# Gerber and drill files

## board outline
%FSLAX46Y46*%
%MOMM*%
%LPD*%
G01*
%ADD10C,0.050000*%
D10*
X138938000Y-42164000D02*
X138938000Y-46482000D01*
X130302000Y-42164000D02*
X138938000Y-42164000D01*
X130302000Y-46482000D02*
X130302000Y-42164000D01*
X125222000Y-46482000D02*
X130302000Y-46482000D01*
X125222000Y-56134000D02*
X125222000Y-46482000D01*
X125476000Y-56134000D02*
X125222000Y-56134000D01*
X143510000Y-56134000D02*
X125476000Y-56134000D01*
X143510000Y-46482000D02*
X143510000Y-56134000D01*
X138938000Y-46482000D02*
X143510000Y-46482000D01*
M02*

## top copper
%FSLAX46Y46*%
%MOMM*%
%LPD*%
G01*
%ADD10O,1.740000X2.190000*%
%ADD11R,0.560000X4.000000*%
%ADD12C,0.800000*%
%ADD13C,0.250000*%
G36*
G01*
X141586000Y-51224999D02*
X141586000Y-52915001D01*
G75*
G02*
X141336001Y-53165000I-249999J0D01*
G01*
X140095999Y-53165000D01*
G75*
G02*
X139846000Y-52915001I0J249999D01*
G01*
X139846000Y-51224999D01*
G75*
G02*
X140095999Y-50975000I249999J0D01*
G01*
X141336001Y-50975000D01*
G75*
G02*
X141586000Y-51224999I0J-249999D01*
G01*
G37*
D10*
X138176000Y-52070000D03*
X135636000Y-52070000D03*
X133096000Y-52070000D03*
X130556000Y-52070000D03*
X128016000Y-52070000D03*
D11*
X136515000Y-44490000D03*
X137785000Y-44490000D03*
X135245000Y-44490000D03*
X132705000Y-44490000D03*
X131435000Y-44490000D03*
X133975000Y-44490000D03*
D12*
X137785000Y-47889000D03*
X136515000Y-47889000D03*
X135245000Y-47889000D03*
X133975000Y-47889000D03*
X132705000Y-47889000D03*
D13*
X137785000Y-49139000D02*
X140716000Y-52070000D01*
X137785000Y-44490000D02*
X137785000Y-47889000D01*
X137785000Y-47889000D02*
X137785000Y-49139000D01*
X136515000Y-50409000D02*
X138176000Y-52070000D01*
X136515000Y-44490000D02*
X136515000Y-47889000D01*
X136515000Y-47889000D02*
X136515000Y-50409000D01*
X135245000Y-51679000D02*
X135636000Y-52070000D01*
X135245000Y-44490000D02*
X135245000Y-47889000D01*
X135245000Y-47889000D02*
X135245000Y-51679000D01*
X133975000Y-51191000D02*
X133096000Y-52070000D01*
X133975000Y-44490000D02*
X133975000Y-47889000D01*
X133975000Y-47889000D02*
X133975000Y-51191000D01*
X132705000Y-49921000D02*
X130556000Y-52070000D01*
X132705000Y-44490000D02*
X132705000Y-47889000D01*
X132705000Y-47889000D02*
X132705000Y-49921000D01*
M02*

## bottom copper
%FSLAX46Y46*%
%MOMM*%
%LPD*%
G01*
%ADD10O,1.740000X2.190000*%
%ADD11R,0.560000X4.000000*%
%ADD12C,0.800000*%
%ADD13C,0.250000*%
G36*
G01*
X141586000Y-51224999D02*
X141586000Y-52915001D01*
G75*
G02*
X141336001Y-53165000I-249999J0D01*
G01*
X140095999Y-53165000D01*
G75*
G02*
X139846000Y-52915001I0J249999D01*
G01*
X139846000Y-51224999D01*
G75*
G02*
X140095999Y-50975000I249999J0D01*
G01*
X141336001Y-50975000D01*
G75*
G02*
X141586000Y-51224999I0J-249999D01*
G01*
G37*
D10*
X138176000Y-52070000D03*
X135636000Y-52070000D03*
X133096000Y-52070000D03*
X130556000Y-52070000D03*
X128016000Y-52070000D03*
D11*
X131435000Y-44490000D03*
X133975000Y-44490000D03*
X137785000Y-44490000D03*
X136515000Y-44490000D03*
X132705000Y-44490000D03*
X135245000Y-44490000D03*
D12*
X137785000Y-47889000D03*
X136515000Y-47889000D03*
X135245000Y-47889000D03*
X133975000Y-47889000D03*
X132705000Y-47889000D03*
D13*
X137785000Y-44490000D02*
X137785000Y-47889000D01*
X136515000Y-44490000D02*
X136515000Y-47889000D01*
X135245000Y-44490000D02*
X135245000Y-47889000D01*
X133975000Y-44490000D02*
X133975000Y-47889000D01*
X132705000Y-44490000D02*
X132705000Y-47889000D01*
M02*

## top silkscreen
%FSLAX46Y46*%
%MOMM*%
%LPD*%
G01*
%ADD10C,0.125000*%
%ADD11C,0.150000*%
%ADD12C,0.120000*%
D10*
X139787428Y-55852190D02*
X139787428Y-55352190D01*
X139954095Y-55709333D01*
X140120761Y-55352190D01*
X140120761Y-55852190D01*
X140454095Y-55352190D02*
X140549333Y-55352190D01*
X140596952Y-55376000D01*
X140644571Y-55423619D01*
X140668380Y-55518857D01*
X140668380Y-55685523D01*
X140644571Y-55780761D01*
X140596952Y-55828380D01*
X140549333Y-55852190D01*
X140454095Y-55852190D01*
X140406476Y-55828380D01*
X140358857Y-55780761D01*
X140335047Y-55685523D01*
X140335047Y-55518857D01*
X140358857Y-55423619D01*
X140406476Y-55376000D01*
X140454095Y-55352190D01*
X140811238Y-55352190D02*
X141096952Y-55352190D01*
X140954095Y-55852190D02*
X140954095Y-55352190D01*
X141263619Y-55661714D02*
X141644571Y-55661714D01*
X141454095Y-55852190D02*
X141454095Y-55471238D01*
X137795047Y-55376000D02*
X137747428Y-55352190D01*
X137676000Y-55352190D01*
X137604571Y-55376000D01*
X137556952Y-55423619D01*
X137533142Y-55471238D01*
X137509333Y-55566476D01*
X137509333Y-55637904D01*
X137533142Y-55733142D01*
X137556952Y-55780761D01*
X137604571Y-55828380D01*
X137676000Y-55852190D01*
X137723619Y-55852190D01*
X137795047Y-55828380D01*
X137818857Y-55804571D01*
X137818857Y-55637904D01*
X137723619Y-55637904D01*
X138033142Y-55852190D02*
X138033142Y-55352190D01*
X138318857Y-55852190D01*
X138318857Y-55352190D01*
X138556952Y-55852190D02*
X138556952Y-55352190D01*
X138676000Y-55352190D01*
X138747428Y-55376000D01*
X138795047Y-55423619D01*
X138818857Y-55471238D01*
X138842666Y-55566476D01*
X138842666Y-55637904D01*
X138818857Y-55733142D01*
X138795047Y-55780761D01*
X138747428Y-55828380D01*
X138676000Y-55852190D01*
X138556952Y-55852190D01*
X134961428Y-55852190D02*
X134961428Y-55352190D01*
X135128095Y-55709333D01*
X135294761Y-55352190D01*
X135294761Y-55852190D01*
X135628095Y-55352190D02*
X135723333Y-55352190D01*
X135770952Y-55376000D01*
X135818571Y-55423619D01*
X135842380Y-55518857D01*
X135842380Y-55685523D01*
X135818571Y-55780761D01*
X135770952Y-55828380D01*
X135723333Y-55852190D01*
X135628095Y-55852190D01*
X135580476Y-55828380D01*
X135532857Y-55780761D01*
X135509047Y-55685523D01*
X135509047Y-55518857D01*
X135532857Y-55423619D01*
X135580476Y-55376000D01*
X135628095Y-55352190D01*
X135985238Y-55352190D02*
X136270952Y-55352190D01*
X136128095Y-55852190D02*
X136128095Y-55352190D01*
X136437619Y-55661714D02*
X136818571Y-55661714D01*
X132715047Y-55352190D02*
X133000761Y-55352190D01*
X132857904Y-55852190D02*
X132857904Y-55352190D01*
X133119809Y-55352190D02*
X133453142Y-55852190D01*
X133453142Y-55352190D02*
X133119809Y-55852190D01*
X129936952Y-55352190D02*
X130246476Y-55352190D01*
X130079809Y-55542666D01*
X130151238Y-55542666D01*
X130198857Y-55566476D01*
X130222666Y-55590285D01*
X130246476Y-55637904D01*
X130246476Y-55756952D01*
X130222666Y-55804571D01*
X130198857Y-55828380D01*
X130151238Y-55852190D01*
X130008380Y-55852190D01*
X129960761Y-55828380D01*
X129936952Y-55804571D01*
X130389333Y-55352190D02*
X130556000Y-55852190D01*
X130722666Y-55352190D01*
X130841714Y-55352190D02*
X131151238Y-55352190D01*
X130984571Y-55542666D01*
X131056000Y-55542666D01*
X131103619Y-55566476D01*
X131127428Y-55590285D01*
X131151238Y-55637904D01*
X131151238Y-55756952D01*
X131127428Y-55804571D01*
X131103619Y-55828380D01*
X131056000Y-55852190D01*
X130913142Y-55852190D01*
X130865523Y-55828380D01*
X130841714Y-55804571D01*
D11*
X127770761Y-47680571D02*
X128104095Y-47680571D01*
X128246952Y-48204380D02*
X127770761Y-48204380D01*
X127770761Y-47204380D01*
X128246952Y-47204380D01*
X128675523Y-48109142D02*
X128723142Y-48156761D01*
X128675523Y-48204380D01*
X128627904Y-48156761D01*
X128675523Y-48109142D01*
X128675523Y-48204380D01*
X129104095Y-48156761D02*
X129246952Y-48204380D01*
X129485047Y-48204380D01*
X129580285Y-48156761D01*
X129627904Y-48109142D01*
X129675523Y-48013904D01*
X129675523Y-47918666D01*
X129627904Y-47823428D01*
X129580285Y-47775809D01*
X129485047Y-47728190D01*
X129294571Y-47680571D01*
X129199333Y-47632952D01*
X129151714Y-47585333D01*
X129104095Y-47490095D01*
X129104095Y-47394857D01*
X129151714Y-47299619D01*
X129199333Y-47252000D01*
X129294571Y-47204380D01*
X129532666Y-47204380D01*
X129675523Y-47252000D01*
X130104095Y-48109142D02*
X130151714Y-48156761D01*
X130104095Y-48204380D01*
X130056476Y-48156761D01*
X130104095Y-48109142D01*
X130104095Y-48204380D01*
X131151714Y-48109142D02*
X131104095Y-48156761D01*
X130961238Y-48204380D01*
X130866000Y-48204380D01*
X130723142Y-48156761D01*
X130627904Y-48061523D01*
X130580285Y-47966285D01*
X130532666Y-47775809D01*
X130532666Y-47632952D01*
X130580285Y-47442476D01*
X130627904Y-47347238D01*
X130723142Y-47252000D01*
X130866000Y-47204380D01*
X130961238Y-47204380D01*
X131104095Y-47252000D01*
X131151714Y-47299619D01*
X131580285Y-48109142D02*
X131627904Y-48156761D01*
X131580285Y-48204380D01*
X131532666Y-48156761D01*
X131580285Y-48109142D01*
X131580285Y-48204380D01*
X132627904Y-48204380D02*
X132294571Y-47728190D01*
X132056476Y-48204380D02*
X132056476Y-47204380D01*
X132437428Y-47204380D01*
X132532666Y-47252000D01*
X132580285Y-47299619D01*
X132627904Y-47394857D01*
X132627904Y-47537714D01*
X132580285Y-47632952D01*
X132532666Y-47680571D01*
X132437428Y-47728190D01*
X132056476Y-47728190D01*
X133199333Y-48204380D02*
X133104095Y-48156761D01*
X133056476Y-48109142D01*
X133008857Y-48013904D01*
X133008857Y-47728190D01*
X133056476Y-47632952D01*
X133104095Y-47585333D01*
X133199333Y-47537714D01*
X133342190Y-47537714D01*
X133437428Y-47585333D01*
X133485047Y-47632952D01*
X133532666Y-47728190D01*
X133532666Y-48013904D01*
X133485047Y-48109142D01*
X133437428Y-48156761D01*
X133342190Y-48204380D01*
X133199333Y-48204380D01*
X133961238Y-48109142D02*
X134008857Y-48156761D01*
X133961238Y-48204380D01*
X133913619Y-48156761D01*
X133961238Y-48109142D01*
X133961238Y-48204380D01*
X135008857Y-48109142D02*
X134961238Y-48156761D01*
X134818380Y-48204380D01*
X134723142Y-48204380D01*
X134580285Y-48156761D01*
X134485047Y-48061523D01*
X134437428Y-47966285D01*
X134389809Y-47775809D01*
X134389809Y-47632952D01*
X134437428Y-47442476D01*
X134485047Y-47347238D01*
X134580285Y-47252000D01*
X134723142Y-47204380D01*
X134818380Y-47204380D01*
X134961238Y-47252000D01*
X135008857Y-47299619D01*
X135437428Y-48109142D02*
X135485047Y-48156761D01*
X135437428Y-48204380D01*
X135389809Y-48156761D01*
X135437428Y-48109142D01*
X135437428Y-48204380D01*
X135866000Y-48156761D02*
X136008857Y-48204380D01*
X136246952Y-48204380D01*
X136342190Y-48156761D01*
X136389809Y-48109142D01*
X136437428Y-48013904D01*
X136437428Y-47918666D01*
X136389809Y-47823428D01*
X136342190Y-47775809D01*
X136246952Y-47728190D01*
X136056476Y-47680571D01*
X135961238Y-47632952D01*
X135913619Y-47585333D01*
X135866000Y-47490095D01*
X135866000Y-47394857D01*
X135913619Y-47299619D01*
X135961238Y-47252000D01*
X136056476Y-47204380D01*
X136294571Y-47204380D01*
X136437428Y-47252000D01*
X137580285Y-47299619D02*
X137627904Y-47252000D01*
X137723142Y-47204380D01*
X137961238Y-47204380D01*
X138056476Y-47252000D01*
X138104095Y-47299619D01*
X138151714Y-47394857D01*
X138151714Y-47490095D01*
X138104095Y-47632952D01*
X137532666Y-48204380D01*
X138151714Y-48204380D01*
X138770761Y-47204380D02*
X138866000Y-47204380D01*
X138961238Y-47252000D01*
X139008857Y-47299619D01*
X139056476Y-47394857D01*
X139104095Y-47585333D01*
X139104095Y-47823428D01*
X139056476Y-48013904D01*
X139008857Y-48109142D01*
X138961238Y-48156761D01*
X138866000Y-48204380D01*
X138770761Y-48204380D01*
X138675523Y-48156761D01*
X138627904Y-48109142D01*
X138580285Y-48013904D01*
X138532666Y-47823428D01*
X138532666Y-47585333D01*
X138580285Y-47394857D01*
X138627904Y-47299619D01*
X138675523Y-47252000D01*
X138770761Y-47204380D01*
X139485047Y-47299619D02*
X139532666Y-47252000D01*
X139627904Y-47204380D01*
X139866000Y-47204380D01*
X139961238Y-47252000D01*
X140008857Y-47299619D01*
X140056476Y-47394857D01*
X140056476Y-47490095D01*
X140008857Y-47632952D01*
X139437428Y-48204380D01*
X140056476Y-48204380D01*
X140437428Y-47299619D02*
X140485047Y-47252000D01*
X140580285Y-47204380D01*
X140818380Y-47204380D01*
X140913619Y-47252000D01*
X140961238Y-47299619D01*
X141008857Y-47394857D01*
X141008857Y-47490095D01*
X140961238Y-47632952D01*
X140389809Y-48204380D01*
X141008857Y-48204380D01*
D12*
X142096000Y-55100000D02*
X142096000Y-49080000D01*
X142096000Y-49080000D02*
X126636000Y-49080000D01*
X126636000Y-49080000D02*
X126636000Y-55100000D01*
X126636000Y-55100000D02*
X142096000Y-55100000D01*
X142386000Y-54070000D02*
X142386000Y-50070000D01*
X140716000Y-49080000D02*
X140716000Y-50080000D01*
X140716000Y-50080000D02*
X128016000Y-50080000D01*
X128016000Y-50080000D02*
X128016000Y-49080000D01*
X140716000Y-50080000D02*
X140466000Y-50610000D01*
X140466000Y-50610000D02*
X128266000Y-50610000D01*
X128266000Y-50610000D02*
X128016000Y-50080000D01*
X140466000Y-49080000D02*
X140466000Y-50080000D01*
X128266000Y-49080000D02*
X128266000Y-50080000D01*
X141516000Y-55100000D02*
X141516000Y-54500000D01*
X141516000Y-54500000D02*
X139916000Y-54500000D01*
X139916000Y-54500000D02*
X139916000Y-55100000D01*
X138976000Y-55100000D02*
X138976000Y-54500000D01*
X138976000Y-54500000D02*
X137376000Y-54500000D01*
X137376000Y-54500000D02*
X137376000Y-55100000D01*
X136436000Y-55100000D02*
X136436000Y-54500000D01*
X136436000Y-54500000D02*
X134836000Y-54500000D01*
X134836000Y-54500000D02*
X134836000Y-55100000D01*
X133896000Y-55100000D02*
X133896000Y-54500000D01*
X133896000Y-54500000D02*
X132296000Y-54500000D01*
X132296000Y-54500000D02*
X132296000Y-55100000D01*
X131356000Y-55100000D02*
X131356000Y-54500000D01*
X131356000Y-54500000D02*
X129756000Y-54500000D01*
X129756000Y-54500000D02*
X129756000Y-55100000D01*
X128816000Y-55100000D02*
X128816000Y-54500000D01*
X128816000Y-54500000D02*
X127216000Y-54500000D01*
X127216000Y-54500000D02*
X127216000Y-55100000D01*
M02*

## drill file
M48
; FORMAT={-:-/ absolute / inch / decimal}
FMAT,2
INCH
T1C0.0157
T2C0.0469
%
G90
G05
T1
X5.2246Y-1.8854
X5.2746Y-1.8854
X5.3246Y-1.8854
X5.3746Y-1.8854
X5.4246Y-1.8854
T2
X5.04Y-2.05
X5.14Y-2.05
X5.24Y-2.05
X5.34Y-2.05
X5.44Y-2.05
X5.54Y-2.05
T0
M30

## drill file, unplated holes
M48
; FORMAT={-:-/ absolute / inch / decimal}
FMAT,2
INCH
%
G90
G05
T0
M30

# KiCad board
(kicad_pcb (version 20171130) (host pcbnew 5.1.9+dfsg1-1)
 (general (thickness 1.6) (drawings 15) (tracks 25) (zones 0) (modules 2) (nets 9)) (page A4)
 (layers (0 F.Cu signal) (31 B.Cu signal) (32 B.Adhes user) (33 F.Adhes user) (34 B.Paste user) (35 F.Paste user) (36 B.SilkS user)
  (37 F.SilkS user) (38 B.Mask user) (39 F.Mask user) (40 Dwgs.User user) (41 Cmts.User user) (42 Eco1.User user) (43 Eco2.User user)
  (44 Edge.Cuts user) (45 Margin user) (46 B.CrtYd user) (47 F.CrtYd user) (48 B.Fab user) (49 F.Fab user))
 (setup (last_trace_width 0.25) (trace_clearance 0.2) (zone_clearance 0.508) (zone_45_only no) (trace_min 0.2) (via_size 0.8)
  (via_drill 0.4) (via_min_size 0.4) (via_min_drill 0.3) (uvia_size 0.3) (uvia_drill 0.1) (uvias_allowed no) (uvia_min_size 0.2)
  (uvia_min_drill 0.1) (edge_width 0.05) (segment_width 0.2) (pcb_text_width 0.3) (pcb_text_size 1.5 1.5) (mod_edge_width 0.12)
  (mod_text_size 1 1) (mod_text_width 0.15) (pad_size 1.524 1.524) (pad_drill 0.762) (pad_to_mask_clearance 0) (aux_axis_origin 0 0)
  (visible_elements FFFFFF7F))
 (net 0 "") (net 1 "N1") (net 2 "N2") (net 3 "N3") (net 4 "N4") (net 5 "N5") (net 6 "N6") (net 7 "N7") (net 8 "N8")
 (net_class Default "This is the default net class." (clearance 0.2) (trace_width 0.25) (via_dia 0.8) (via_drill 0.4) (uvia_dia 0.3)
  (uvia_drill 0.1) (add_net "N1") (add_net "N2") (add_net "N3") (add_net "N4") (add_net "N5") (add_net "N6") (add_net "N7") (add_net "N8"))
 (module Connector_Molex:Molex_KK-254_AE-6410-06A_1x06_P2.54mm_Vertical (layer F.Cu) (at 140.716 52.07 180)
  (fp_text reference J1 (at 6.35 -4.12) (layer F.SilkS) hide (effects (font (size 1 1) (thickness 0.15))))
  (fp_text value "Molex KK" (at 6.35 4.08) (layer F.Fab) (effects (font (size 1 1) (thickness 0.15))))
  (fp_line (start 13.5 -2.43) (end 13.5 -3.03) (layer F.SilkS) (width 0.12))
  (fp_line (start 11.9 -2.43) (end 13.5 -2.43) (layer F.SilkS) (width 0.12))
  (fp_line (start 11.9 -3.03) (end 11.9 -2.43) (layer F.SilkS) (width 0.12))
  (fp_line (start 10.96 -2.43) (end 10.96 -3.03) (layer F.SilkS) (width 0.12))
  (fp_line (start 9.36 -2.43) (end 10.96 -2.43) (layer F.SilkS) (width 0.12))
  (fp_line (start 9.36 -3.03) (end 9.36 -2.43) (layer F.SilkS) (width 0.12))
  (fp_line (start 8.42 -2.43) (end 8.42 -3.03) (layer F.SilkS) (width 0.12))
  (fp_line (start 6.82 -2.43) (end 8.42 -2.43) (layer F.SilkS) (width 0.12))
  (fp_line (start 6.82 -3.03) (end 6.82 -2.43) (layer F.SilkS) (width 0.12))
  (fp_line (start 5.88 -2.43) (end 5.88 -3.03) (layer F.SilkS) (width 0.12))
  (fp_line (start 4.28 -2.43) (end 5.88 -2.43) (layer F.SilkS) (width 0.12))
  (fp_line (start 4.28 -3.03) (end 4.28 -2.43) (layer F.SilkS) (width 0.12))
  (fp_line (start 3.34 -2.43) (end 3.34 -3.03) (layer F.SilkS) (width 0.12))
  (fp_line (start 1.74 -2.43) (end 3.34 -2.43) (layer F.SilkS) (width 0.12))
  (fp_line (start 1.74 -3.03) (end 1.74 -2.43) (layer F.SilkS) (width 0.12))
  (fp_line (start 0.8 -2.43) (end 0.8 -3.03) (layer F.SilkS) (width 0.12))
  (fp_line (start -0.8 -2.43) (end 0.8 -2.43) (layer F.SilkS) (width 0.12))
  (fp_line (start -0.8 -3.03) (end -0.8 -2.43) (layer F.SilkS) (width 0.12))
  (fp_line (start 12.45 2.99) (end 12.45 1.99) (layer F.SilkS) (width 0.12))
  (fp_line (start 0.25 2.99) (end 0.25 1.99) (layer F.SilkS) (width 0.12))
  (fp_line (start 12.45 1.46) (end 12.7 1.99) (layer F.SilkS) (width 0.12))
  (fp_line (start 0.25 1.46) (end 12.45 1.46) (layer F.SilkS) (width 0.12))
  (fp_line (start 0 1.99) (end 0.25 1.46) (layer F.SilkS) (width 0.12))
  (fp_line (start 12.7 1.99) (end 12.7 2.99) (layer F.SilkS) (width 0.12))
  (fp_line (start 0 1.99) (end 12.7 1.99) (layer F.SilkS) (width 0.12))
  (fp_line (start 0 2.99) (end 0 1.99) (layer F.SilkS) (width 0.12))
  (fp_line (start -1.67 -2) (end -1.67 2) (layer F.SilkS) (width 0.12))
  (fp_line (start 14.08 -3.03) (end -1.38 -3.03) (layer F.SilkS) (width 0.12))
  (fp_line (start 14.08 2.99) (end 14.08 -3.03) (layer F.SilkS) (width 0.12))
  (fp_line (start -1.38 2.99) (end 14.08 2.99) (layer F.SilkS) (width 0.12))
  (fp_line (start -1.38 -3.03) (end -1.38 2.99) (layer F.SilkS) (width 0.12))
  (pad 1 thru_hole roundrect (at 0 0 180) (size 1.74 2.19) (drill 1.19) (layers *.Cu *.Mask) (roundrect_rratio 0.1436775862068966)
   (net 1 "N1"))
  (pad 2 thru_hole oval (at 2.54 0 180) (size 1.74 2.19) (drill 1.19) (layers *.Cu *.Mask) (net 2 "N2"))
  (pad 3 thru_hole oval (at 5.08 0 180) (size 1.74 2.19) (drill 1.19) (layers *.Cu *.Mask) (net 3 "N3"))
  (pad 4 thru_hole oval (at 7.62 0 180) (size 1.74 2.19) (drill 1.19) (layers *.Cu *.Mask) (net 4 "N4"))
  (pad 5 thru_hole oval (at 10.16 0 180) (size 1.74 2.19) (drill 1.19) (layers *.Cu *.Mask) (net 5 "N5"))
  (pad 6 thru_hole oval (at 12.7 0 180) (size 1.74 2.19) (drill 1.19) (layers *.Cu *.Mask) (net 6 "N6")))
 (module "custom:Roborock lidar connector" (layer F.Cu) (at 134.62 44.704 180)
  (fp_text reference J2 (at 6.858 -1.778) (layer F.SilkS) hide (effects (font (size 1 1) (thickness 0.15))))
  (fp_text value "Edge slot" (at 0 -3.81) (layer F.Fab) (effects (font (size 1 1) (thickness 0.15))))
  (pad 3 connect rect (at -1.895 0.214 180) (size 0.56 4) (layers F.Cu F.Mask) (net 2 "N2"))
  (pad 1 connect rect (at -3.165 0.214 180) (size 0.56 4) (layers F.Cu F.Mask) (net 1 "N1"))
  (pad 5 connect rect (at -0.625 0.214 180) (size 0.56 4) (layers F.Cu F.Mask) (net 3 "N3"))
  (pad 9 connect rect (at 1.915 0.214 180) (size 0.56 4) (layers F.Cu F.Mask) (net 5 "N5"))
  (pad 11 connect rect (at 3.185 0.214 180) (size 0.56 4) (layers F.Cu F.Mask) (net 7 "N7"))
  (pad 12 connect rect (at 3.185 0.214 180) (size 0.56 4) (layers B.Cu B.Mask) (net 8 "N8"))
  (pad 8 connect rect (at 0.645 0.214 180) (size 0.56 4) (layers B.Cu B.Mask) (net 4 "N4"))
  (pad 2 connect rect (at -3.165 0.214 180) (size 0.56 4) (layers B.Cu B.Mask) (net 1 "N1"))
  (pad 4 connect rect (at -1.895 0.214 180) (size 0.56 4) (layers B.Cu B.Mask) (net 2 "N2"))
  (pad 10 connect rect (at 1.915 0.214 180) (size 0.56 4) (layers B.Cu B.Mask) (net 5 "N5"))
  (pad 7 connect rect (at 0.645 0.214 180) (size 0.56 4) (layers F.Cu F.Mask) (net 4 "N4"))
  (pad 6 connect rect (at -0.625 0.214 180) (size 0.56 4) (layers B.Cu B.Mask) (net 3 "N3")))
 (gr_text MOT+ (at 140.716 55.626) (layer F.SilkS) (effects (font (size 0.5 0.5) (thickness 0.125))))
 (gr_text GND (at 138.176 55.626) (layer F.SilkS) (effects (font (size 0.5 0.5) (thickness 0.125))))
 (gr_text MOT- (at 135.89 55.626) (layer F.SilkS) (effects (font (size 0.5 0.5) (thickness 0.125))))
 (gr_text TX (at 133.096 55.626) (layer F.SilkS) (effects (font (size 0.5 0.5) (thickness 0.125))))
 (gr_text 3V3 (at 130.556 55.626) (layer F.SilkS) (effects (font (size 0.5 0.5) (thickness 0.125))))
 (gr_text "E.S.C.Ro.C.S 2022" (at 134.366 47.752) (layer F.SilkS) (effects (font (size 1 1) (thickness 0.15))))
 (gr_line (start 138.938 42.164) (end 138.938 46.482) (layer Edge.Cuts) (width 0.05))
 (gr_line (start 130.302 42.164) (end 138.938 42.164) (layer Edge.Cuts) (width 0.05))
 (gr_line (start 130.302 46.482) (end 130.302 42.164) (layer Edge.Cuts) (width 0.05))
 (gr_line (start 125.222 46.482) (end 130.302 46.482) (layer Edge.Cuts) (width 0.05))
 (gr_line (start 125.222 56.134) (end 125.222 46.482) (layer Edge.Cuts) (width 0.05))
 (gr_line (start 125.476 56.134) (end 125.222 56.134) (layer Edge.Cuts) (width 0.05))
 (gr_line (start 143.51 56.134) (end 125.476 56.134) (layer Edge.Cuts) (width 0.05))
 (gr_line (start 143.51 46.482) (end 143.51 56.134) (layer Edge.Cuts) (width 0.05))
 (gr_line (start 138.938 46.482) (end 143.51 46.482) (layer Edge.Cuts) (width 0.05))
 (segment (start 137.785 49.139) (end 140.716 52.07) (width 0.25) (layer F.Cu) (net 1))
 (segment (start 137.785 44.49) (end 137.785 47.889) (width 0.25) (layer F.Cu) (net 1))
 (segment (start 137.785 47.889) (end 137.785 49.139) (width 0.25) (layer F.Cu) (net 1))
 (via (at 137.785 47.889) (size 0.8) (drill 0.4) (layers F.Cu B.Cu) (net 1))
 (segment (start 137.785 44.49) (end 137.785 47.889) (width 0.25) (layer B.Cu) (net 1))
 (segment (start 136.515 50.409) (end 138.176 52.07) (width 0.25) (layer F.Cu) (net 2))
 (segment (start 136.515 44.49) (end 136.515 47.889) (width 0.25) (layer F.Cu) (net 2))
 (segment (start 136.515 47.889) (end 136.515 50.409) (width 0.25) (layer F.Cu) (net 2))
 (via (at 136.515 47.889) (size 0.8) (drill 0.4) (layers F.Cu B.Cu) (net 2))
 (segment (start 136.515 44.49) (end 136.515 47.889) (width 0.25) (layer B.Cu) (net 2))
 (segment (start 135.245 51.679) (end 135.636 52.07) (width 0.25) (layer F.Cu) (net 3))
 (segment (start 135.245 44.49) (end 135.245 47.889) (width 0.25) (layer F.Cu) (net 3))
 (segment (start 135.245 47.889) (end 135.245 51.679) (width 0.25) (layer F.Cu) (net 3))
 (via (at 135.245 47.889) (size 0.8) (drill 0.4) (layers F.Cu B.Cu) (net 3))
 (segment (start 135.245 44.49) (end 135.245 47.889) (width 0.25) (layer B.Cu) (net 3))
 (segment (start 133.975 51.191) (end 133.096 52.07) (width 0.25) (layer F.Cu) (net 4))
 (segment (start 133.975 44.49) (end 133.975 47.889) (width 0.25) (layer F.Cu) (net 4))
 (segment (start 133.975 47.889) (end 133.975 51.191) (width 0.25) (layer F.Cu) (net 4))
 (via (at 133.975 47.889) (size 0.8) (drill 0.4) (layers F.Cu B.Cu) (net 4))
 (segment (start 133.975 44.49) (end 133.975 47.889) (width 0.25) (layer B.Cu) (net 4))
 (segment (start 132.705 49.921) (end 130.556 52.07) (width 0.25) (layer F.Cu) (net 5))
 (segment (start 132.705 44.49) (end 132.705 47.889) (width 0.25) (layer F.Cu) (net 5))
 (segment (start 132.705 47.889) (end 132.705 49.921) (width 0.25) (layer F.Cu) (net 5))
 (via (at 132.705 47.889) (size 0.8) (drill 0.4) (layers F.Cu B.Cu) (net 5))
 (segment (start 132.705 44.49) (end 132.705 47.889) (width 0.25) (layer B.Cu) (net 5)))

